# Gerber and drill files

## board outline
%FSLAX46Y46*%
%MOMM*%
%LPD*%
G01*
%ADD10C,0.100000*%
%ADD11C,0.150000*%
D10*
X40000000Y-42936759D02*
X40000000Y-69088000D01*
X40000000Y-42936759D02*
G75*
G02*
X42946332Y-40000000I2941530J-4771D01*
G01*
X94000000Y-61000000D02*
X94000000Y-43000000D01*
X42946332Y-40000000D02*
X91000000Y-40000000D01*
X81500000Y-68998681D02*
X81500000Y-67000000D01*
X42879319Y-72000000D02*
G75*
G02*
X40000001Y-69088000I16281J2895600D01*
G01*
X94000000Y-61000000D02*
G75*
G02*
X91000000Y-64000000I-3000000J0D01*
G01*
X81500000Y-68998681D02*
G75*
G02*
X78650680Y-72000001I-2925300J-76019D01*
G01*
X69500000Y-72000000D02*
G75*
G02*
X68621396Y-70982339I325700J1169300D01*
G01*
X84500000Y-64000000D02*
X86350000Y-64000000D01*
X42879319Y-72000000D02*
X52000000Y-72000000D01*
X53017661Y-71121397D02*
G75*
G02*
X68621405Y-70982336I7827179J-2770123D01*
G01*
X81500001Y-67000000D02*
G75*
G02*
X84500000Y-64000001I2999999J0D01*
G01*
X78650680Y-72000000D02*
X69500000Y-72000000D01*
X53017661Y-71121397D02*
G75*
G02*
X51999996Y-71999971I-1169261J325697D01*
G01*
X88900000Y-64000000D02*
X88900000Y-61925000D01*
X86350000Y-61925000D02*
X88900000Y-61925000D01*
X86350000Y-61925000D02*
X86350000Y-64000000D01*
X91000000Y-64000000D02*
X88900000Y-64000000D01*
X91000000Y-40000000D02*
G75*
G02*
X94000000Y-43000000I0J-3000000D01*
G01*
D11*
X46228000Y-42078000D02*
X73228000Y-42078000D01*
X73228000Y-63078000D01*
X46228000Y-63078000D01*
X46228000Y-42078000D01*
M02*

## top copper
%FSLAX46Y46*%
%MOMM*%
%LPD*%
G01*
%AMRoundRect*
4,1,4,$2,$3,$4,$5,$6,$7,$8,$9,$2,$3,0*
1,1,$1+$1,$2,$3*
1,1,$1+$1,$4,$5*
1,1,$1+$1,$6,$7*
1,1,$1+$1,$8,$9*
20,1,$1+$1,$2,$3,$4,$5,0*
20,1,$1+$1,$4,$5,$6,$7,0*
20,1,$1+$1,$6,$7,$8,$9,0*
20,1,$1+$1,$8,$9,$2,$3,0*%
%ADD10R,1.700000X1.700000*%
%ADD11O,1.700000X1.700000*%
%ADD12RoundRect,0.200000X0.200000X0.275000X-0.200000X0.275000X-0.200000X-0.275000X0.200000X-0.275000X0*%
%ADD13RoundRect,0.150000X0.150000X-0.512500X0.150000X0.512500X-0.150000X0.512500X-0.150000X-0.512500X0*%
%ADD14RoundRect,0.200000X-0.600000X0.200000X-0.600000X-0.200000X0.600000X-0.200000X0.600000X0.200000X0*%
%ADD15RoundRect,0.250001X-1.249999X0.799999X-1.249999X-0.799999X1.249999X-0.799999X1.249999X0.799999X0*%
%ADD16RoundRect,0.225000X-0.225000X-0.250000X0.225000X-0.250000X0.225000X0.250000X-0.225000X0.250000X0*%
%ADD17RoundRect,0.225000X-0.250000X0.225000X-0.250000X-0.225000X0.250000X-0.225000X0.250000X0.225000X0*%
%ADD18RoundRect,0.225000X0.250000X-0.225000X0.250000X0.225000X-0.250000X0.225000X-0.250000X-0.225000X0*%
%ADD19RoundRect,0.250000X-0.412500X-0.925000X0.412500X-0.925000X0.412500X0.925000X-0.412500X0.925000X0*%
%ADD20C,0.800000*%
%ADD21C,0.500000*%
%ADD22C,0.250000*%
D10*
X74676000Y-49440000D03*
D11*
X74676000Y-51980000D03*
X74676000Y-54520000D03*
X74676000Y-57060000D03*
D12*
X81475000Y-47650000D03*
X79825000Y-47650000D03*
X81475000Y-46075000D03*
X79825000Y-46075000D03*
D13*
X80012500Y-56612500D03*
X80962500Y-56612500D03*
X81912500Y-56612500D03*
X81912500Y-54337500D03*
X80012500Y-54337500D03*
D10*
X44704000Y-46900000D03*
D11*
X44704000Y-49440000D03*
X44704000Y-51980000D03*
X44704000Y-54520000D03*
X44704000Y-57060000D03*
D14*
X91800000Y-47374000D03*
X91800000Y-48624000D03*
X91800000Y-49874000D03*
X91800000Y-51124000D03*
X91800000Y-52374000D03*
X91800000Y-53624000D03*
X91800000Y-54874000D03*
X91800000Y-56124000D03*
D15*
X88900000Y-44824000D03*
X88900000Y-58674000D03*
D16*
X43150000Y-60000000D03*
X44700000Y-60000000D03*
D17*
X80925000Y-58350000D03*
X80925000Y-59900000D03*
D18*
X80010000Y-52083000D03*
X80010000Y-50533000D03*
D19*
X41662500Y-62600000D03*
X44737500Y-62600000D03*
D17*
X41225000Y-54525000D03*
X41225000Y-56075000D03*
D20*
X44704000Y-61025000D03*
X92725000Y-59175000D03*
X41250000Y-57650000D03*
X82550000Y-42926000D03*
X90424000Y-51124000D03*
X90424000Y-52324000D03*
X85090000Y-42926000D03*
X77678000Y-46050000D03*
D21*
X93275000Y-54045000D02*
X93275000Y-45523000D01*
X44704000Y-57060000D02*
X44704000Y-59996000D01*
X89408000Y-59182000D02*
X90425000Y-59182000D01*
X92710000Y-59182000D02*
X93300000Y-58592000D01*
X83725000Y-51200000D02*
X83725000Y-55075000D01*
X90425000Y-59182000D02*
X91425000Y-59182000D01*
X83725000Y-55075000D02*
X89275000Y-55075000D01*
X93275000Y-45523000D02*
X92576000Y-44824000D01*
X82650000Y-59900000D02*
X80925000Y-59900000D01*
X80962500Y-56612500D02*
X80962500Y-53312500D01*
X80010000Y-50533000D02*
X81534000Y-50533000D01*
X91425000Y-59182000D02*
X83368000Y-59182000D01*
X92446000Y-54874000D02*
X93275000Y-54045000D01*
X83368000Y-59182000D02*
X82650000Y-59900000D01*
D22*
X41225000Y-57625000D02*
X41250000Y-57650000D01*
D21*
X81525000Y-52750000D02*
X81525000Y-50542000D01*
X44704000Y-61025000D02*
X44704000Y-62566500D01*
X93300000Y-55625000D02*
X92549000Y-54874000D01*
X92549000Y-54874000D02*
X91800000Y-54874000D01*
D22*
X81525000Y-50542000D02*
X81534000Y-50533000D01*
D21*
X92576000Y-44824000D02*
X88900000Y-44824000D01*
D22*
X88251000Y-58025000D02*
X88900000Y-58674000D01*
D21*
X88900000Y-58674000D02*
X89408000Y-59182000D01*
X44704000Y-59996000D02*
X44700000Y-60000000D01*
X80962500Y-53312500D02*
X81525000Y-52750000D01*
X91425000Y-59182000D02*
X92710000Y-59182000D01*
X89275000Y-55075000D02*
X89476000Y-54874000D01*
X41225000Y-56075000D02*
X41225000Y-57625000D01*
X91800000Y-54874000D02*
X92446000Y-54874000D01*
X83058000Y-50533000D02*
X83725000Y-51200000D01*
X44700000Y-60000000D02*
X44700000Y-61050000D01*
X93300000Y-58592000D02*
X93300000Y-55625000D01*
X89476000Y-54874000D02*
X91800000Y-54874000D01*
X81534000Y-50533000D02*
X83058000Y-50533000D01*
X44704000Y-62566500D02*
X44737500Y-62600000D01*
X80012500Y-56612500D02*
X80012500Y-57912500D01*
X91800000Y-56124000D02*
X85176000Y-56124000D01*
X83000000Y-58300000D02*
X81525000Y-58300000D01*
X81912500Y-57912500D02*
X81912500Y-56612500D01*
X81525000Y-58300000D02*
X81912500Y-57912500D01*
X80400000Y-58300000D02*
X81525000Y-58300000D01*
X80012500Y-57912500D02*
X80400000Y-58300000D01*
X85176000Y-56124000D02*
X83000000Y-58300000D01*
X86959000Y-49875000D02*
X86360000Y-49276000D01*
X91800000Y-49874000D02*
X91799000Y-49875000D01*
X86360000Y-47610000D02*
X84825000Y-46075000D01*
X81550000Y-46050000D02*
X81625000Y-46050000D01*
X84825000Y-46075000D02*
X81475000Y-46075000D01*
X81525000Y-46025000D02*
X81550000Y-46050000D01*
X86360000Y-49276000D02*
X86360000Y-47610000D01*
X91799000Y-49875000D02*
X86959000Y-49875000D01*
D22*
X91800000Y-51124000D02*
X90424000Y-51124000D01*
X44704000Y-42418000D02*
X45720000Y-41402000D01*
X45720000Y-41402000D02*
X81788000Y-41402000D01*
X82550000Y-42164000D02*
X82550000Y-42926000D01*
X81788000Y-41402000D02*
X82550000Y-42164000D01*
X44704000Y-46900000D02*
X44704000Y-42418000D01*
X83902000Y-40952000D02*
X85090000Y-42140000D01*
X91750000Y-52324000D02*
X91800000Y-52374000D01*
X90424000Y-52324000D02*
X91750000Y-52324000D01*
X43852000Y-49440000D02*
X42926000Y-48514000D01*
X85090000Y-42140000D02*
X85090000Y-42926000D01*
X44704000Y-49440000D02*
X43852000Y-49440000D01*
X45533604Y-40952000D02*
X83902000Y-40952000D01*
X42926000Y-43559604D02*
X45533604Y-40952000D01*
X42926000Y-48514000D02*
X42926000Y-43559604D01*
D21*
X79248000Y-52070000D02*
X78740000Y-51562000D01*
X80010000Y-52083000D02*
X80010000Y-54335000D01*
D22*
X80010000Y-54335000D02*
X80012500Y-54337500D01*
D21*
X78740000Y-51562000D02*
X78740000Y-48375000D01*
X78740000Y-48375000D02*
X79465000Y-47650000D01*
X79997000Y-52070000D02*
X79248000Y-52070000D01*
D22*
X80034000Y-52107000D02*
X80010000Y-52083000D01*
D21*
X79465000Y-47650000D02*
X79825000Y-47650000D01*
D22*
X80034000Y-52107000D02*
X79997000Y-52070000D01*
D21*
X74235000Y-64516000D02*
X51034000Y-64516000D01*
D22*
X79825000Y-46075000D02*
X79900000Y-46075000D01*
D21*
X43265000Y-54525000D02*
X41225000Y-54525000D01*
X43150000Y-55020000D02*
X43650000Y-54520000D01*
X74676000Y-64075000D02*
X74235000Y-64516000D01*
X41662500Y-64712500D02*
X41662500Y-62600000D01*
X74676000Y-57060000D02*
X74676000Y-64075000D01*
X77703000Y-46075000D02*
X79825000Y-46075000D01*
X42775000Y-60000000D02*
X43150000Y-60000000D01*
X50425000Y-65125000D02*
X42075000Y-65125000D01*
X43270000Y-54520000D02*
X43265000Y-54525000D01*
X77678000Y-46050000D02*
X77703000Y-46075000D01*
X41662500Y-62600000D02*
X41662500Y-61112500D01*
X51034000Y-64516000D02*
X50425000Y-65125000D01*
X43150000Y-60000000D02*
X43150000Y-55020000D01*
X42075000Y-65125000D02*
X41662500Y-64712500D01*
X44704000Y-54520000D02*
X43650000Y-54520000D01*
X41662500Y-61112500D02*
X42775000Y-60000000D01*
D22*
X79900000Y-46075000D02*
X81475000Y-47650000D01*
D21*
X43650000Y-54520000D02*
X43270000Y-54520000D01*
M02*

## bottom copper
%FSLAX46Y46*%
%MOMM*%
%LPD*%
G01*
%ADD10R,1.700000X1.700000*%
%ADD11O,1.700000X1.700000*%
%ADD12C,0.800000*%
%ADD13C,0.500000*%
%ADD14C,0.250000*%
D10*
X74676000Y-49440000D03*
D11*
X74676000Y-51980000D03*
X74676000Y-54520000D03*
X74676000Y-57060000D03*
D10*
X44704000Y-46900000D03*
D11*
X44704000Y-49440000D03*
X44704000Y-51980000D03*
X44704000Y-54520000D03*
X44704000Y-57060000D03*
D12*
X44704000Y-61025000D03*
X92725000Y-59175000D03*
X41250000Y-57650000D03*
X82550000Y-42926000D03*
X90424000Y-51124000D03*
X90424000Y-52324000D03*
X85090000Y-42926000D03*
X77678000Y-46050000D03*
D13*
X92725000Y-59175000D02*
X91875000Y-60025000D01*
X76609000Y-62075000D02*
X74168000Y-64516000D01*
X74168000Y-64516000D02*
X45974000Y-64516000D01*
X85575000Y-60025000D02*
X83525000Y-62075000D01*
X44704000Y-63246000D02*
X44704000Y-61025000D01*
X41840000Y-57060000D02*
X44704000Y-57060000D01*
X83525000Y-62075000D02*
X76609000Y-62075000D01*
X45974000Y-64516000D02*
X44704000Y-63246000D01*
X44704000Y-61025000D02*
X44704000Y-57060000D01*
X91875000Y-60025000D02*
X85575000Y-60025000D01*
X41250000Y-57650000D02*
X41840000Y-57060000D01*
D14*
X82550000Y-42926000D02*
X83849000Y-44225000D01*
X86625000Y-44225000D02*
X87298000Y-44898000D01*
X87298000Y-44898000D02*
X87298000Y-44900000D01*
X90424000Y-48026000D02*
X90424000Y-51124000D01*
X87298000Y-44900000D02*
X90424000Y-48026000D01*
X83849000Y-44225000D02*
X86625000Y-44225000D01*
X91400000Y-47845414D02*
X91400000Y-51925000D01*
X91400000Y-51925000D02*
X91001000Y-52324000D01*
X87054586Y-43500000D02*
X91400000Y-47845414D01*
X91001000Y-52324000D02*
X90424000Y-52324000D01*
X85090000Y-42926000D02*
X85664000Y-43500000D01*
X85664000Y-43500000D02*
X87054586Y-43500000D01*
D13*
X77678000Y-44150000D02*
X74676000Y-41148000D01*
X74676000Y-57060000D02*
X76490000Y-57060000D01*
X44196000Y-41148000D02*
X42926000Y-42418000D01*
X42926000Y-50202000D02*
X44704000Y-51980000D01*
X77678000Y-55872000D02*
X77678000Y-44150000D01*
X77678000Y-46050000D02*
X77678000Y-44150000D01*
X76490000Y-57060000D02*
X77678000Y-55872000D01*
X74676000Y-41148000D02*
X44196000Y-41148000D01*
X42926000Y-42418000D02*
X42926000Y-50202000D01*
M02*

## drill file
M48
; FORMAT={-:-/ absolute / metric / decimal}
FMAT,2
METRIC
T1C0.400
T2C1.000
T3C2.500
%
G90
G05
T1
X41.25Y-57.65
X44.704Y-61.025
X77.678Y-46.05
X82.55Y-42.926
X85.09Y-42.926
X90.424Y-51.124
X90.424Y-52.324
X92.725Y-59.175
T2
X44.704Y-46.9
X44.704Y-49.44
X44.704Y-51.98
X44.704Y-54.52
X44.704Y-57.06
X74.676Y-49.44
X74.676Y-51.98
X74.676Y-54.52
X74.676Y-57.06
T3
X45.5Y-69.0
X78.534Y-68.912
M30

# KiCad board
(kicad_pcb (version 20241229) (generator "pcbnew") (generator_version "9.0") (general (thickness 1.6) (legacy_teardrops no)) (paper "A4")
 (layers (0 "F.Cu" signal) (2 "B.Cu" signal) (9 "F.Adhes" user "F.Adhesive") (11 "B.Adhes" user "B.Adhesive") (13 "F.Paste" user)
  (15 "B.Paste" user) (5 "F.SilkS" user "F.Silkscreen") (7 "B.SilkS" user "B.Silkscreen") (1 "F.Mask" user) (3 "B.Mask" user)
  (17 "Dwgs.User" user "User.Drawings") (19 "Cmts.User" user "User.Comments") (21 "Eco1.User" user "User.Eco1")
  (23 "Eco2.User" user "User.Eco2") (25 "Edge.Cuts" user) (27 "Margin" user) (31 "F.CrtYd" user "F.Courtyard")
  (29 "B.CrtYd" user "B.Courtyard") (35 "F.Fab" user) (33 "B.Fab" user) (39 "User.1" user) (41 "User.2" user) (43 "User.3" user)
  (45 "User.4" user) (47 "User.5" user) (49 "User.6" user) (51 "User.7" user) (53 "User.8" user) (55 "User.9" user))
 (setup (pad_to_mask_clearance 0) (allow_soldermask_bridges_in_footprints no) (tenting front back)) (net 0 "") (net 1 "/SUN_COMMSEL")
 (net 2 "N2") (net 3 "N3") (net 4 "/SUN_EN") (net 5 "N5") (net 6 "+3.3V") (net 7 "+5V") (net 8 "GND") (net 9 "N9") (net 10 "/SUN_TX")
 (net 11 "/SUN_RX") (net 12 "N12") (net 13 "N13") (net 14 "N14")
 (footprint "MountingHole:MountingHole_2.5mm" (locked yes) (layer "F.Cu") (at 45.466 69.088)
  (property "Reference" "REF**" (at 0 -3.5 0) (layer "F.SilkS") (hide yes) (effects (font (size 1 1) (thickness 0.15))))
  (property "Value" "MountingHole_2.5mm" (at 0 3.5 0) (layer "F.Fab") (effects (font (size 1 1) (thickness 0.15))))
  (pad "" np_thru_hole circle (at 0.034 -0.088) (size 2.5 2.5) (drill 2.5) (layers "*.Cu" "*.Mask")))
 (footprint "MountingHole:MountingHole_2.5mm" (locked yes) (layer "F.Cu") (at 78.5 69)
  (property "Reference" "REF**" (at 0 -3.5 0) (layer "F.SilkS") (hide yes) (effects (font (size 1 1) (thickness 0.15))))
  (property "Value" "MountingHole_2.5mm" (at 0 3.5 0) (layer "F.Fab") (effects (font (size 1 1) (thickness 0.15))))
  (pad "" np_thru_hole circle (at 0.034 -0.088) (size 2.5 2.5) (drill 2.5) (layers "*.Cu" "*.Mask")))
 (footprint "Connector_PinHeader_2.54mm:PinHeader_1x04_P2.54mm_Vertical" (layer "F.Cu") (at 74.676 49.44)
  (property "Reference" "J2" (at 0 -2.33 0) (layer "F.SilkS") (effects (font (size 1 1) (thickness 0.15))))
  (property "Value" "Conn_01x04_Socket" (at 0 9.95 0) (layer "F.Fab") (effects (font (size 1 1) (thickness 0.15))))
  (pad "1" thru_hole rect (at 0 0) (size 1.7 1.7) (drill 1) (layers "*.Cu" "*.Mask") (remove_unused_layers no) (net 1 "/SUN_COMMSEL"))
  (pad "2" thru_hole oval (at 0 2.54) (size 1.7 1.7) (drill 1) (layers "*.Cu" "*.Mask") (remove_unused_layers no) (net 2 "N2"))
  (pad "3" thru_hole oval (at 0 5.08) (size 1.7 1.7) (drill 1) (layers "*.Cu" "*.Mask") (remove_unused_layers no) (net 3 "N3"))
  (pad "4" thru_hole oval (at 0 7.62) (size 1.7 1.7) (drill 1) (layers "*.Cu" "*.Mask") (remove_unused_layers no) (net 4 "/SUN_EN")))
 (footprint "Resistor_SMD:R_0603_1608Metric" (layer "F.Cu") (at 80.65 47.65 180)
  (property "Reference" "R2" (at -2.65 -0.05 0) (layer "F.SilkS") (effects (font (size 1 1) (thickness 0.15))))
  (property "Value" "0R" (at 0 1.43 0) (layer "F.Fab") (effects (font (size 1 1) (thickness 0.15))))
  (pad "1" smd roundrect (at -0.825 0 180) (size 0.8 0.95) (layers "F.Cu" "F.Mask" "F.Paste") (roundrect_rratio 0.25) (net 4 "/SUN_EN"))
  (pad "2" smd roundrect (at 0.825 0 180) (size 0.8 0.95) (layers "F.Cu" "F.Mask" "F.Paste") (roundrect_rratio 0.25) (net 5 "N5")))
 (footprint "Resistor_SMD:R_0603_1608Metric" (layer "F.Cu") (at 80.65 46.075 180)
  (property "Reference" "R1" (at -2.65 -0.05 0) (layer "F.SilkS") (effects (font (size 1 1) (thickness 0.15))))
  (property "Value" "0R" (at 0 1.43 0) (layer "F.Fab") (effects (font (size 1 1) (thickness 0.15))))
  (pad "1" smd roundrect (at -0.825 0 180) (size 0.8 0.95) (layers "F.Cu" "F.Mask" "F.Paste") (roundrect_rratio 0.25) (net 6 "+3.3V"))
  (pad "2" smd roundrect (at 0.825 0 180) (size 0.8 0.95) (layers "F.Cu" "F.Mask" "F.Paste") (roundrect_rratio 0.25) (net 4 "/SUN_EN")))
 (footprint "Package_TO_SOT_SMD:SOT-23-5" (layer "F.Cu") (at 80.9625 55.475 90)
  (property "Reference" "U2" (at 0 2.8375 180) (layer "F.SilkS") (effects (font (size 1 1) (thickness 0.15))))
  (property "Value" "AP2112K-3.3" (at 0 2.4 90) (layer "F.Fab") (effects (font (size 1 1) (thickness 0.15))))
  (pad "1" smd roundrect (at -1.1375 -0.95 90) (size 1.325 0.6) (layers "F.Cu" "F.Mask" "F.Paste") (roundrect_rratio 0.25) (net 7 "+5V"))
  (pad "2" smd roundrect (at -1.1375 0 90) (size 1.325 0.6) (layers "F.Cu" "F.Mask" "F.Paste") (roundrect_rratio 0.25) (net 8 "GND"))
  (pad "3" smd roundrect (at -1.1375 0.95 90) (size 1.325 0.6) (layers "F.Cu" "F.Mask" "F.Paste") (roundrect_rratio 0.25) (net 7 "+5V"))
  (pad "4" smd roundrect (at 1.1375 0.95 90) (size 1.325 0.6) (layers "F.Cu" "F.Mask" "F.Paste") (roundrect_rratio 0.25) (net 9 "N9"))
  (pad "5" smd roundrect (at 1.1375 -0.95 90) (size 1.325 0.6) (layers "F.Cu" "F.Mask" "F.Paste") (roundrect_rratio 0.25) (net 5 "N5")))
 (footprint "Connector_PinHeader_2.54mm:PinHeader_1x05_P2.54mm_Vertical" (layer "F.Cu") (at 44.704 46.9)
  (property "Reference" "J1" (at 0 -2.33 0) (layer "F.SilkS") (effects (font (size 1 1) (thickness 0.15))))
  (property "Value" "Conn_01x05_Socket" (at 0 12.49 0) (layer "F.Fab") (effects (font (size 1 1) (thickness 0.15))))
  (pad "1" thru_hole rect (at 0 0) (size 1.7 1.7) (drill 1) (layers "*.Cu" "*.Mask") (remove_unused_layers no) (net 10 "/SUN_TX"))
  (pad "2" thru_hole oval (at 0 2.54) (size 1.7 1.7) (drill 1) (layers "*.Cu" "*.Mask") (remove_unused_layers no) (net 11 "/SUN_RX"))
  (pad "3" thru_hole oval (at 0 5.08) (size 1.7 1.7) (drill 1) (layers "*.Cu" "*.Mask") (remove_unused_layers no) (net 4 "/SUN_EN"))
  (pad "4" thru_hole oval (at 0 7.62) (size 1.7 1.7) (drill 1) (layers "*.Cu" "*.Mask") (remove_unused_layers no) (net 4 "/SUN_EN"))
  (pad "5" thru_hole oval (at 0 10.16) (size 1.7 1.7) (drill 1) (layers "*.Cu" "*.Mask") (remove_unused_layers no) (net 8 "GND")))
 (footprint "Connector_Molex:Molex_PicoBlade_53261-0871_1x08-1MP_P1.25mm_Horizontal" (layer "F.Cu") (at 89.4 51.749 -90)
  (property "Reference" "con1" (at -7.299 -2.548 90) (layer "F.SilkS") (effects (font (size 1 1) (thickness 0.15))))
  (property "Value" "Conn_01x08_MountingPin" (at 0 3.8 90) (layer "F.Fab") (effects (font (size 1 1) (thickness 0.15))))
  (pad "1" smd roundrect (at -4.375 -2.4 270) (size 0.8 1.6) (layers "F.Cu" "F.Mask" "F.Paste") (roundrect_rratio 0.25) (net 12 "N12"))
  (pad "2" smd roundrect (at -3.125 -2.4 270) (size 0.8 1.6) (layers "F.Cu" "F.Mask" "F.Paste") (roundrect_rratio 0.25) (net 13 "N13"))
  (pad "3" smd roundrect (at -1.875 -2.4 270) (size 0.8 1.6) (layers "F.Cu" "F.Mask" "F.Paste") (roundrect_rratio 0.25) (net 6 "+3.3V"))
  (pad "4" smd roundrect (at -0.625 -2.4 270) (size 0.8 1.6) (layers "F.Cu" "F.Mask" "F.Paste") (roundrect_rratio 0.25) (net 10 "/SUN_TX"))
  (pad "5" smd roundrect (at 0.625 -2.4 270) (size 0.8 1.6) (layers "F.Cu" "F.Mask" "F.Paste") (roundrect_rratio 0.25) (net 11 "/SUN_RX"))
  (pad "6" smd roundrect (at 1.875 -2.4 270) (size 0.8 1.6) (layers "F.Cu" "F.Mask" "F.Paste") (roundrect_rratio 0.25) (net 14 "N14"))
  (pad "7" smd roundrect (at 3.125 -2.4 270) (size 0.8 1.6) (layers "F.Cu" "F.Mask" "F.Paste") (roundrect_rratio 0.25) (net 8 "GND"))
  (pad "8" smd roundrect (at 4.375 -2.4 270) (size 0.8 1.6) (layers "F.Cu" "F.Mask" "F.Paste") (roundrect_rratio 0.25) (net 7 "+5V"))
  (pad "MP" smd roundrect (at -6.925 0.5 270) (size 2.1 3) (layers "F.Cu" "F.Mask" "F.Paste") (roundrect_rratio 0.1190480952) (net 8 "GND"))
  (pad "MP" smd roundrect (at 6.925 0.5 270) (size 2.1 3) (layers "F.Cu" "F.Mask" "F.Paste") (roundrect_rratio 0.1190480952) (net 8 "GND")))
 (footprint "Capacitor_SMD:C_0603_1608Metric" (layer "F.Cu") (at 43.925 60)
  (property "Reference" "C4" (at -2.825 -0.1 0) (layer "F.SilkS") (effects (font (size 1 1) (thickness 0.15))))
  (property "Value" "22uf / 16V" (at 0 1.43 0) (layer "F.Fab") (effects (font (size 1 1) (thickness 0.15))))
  (pad "1" smd roundrect (at -0.775 0) (size 0.9 0.95) (layers "F.Cu" "F.Mask" "F.Paste") (roundrect_rratio 0.25) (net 4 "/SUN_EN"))
  (pad "2" smd roundrect (at 0.775 0) (size 0.9 0.95) (layers "F.Cu" "F.Mask" "F.Paste") (roundrect_rratio 0.25) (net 8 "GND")))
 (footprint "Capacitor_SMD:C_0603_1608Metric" (layer "F.Cu") (at 80.925 59.125 -90)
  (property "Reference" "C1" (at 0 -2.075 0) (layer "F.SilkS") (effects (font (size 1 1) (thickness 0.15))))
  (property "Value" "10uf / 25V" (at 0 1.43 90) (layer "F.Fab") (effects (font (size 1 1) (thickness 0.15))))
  (pad "1" smd roundrect (at -0.775 0 270) (size 0.9 0.95) (layers "F.Cu" "F.Mask" "F.Paste") (roundrect_rratio 0.25) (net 7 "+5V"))
  (pad "2" smd roundrect (at 0.775 0 270) (size 0.9 0.95) (layers "F.Cu" "F.Mask" "F.Paste") (roundrect_rratio 0.25) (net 8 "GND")))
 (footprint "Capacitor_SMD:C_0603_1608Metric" (layer "F.Cu") (at 80.01 51.308 90)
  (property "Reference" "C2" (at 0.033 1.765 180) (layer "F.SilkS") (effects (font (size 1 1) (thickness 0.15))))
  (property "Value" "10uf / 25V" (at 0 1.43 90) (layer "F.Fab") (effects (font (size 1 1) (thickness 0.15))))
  (pad "1" smd roundrect (at -0.775 0 90) (size 0.9 0.95) (layers "F.Cu" "F.Mask" "F.Paste") (roundrect_rratio 0.25) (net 5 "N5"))
  (pad "2" smd roundrect (at 0.775 0 90) (size 0.9 0.95) (layers "F.Cu" "F.Mask" "F.Paste") (roundrect_rratio 0.25) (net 8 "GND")))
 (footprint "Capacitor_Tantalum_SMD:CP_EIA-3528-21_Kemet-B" (layer "F.Cu") (at 43.2 62.6)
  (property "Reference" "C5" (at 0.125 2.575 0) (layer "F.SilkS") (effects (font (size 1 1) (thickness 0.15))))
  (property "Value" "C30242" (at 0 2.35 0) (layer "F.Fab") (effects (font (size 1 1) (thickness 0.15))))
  (pad "1" smd roundrect (at -1.5375 0) (size 1.325 2.35) (layers "F.Cu" "F.Mask" "F.Paste") (roundrect_rratio 0.188679) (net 4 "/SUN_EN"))
  (pad "2" smd roundrect (at 1.5375 0) (size 1.325 2.35) (layers "F.Cu" "F.Mask" "F.Paste") (roundrect_rratio 0.188679) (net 8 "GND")))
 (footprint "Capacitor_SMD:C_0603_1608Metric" (layer "F.Cu") (at 41.225 55.3 -90)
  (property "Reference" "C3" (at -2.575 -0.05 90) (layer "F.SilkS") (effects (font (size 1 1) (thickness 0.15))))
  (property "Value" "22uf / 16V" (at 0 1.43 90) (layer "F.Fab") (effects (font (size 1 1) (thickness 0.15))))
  (pad "1" smd roundrect (at -0.775 0 270) (size 0.9 0.95) (layers "F.Cu" "F.Mask" "F.Paste") (roundrect_rratio 0.25) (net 4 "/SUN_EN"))
  (pad "2" smd roundrect (at 0.775 0 270) (size 0.9 0.95) (layers "F.Cu" "F.Mask" "F.Paste") (roundrect_rratio 0.25) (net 8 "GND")))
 (gr_line (start 40 42.936759) (end 40 69.088) (stroke (width 0.1) (type default)) (locked yes) (layer "Edge.Cuts"))
 (gr_arc (start 40 42.936759) (mid 40.864938 40.858169) (end 42.946332 40) (stroke (width 0.1) (type default)) (locked yes)
  (layer "Edge.Cuts"))
 (gr_line (start 94 61) (end 94 43) (stroke (width 0.1) (type default)) (locked yes) (layer "Edge.Cuts"))
 (gr_line (start 42.946332 40) (end 91 40) (stroke (width 0.1) (type default)) (locked yes) (layer "Edge.Cuts"))
 (gr_line (start 81.5 68.998681) (end 81.5 67) (stroke (width 0.1) (type default)) (locked yes) (layer "Edge.Cuts"))
 (gr_arc (start 42.879319 72) (mid 40.83656 71.140332) (end 40 69.088) (stroke (width 0.1) (type default)) (locked yes) (layer "Edge.Cuts"))
 (gr_arc (start 94 61) (mid 93.121321 63.121321) (end 91 64) (stroke (width 0.1) (type default)) (locked yes) (layer "Edge.Cuts"))
 (gr_arc (start 81.5 68.998681) (mid 80.696939 71.089459) (end 78.65068 72) (stroke (width 0.1) (type default)) (locked yes)
  (layer "Edge.Cuts"))
 (gr_arc (start 69.5 72) (mid 68.906927 71.623929) (end 68.621397 70.982339) (stroke (width 0.1) (type default)) (locked yes)
  (layer "Edge.Cuts"))
 (gr_line (start 84.5 64) (end 86.35 64) (stroke (width 0.1) (type default)) (locked yes) (layer "Edge.Cuts"))
 (gr_line (start 42.879319 72) (end 52 72) (stroke (width 0.1) (type default)) (locked yes) (layer "Edge.Cuts"))
 (gr_arc (start 53.017661 71.121397) (mid 60.770843 65.588942) (end 68.621397 70.982339) (stroke (width 0.1) (type default)) (locked yes)
  (layer "Edge.Cuts"))
 (gr_arc (start 81.500001 67) (mid 82.37868 64.878681) (end 84.5 64) (stroke (width 0.1) (type default)) (locked yes) (layer "Edge.Cuts"))
 (gr_line (start 78.65068 72) (end 69.5 72) (stroke (width 0.1) (type default)) (locked yes) (layer "Edge.Cuts"))
 (gr_arc (start 53.017661 71.121397) (mid 52.64159 71.71447) (end 52 72) (stroke (width 0.1) (type default)) (locked yes)
  (layer "Edge.Cuts"))
 (gr_line (start 88.9 64) (end 88.9 61.925) (stroke (width 0.1) (type default)) (locked yes) (layer "Edge.Cuts"))
 (gr_line (start 86.35 61.925) (end 88.9 61.925) (stroke (width 0.1) (type default)) (locked yes) (layer "Edge.Cuts"))
 (gr_line (start 86.35 61.925) (end 86.35 64) (stroke (width 0.1) (type default)) (locked yes) (layer "Edge.Cuts"))
 (gr_line (start 91 64) (end 88.9 64) (stroke (width 0.1) (type default)) (locked yes) (layer "Edge.Cuts"))
 (gr_arc (start 91 40) (mid 93.121321 40.878679) (end 94 43) (stroke (width 0.1) (type default)) (locked yes) (layer "Edge.Cuts"))
 (gr_rect (start 46.228 42.078) (end 73.228 63.078) (stroke (width 0.15) (type default)) (fill no) (locked yes) (layer "Edge.Cuts"))
 (segment (start 93.275 54.045) (end 93.275 45.523) (width 0.5) (layer "F.Cu") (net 8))
 (segment (start 44.704 57.06) (end 44.704 59.996) (width 0.5) (layer "F.Cu") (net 8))
 (segment (start 89.408 59.182) (end 90.425 59.182) (width 0.5) (layer "F.Cu") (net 8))
 (segment (start 92.71 59.182) (end 93.3 58.592) (width 0.5) (layer "F.Cu") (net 8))
 (segment (start 83.725 51.2) (end 83.725 55.075) (width 0.5) (layer "F.Cu") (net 8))
 (segment (start 90.425 59.182) (end 91.425 59.182) (width 0.5) (layer "F.Cu") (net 8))
 (segment (start 83.725 55.075) (end 89.275 55.075) (width 0.5) (layer "F.Cu") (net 8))
 (segment (start 93.275 45.523) (end 92.576 44.824) (width 0.5) (layer "F.Cu") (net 8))
 (segment (start 82.65 59.9) (end 80.925 59.9) (width 0.5) (layer "F.Cu") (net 8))
 (segment (start 80.9625 56.6125) (end 80.9625 53.3125) (width 0.5) (layer "F.Cu") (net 8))
 (segment (start 80.01 50.533) (end 81.534 50.533) (width 0.5) (layer "F.Cu") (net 8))
 (segment (start 91.425 59.182) (end 83.368 59.182) (width 0.5) (layer "F.Cu") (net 8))
 (segment (start 92.446 54.874) (end 93.275 54.045) (width 0.5) (layer "F.Cu") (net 8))
 (segment (start 83.368 59.182) (end 82.65 59.9) (width 0.5) (layer "F.Cu") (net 8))
 (segment (start 41.225 57.625) (end 41.25 57.65) (width 0.25) (layer "F.Cu") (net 8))
 (segment (start 81.525 52.75) (end 81.525 50.542) (width 0.5) (layer "F.Cu") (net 8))
 (segment (start 44.704 61.025) (end 44.704 62.5665) (width 0.5) (layer "F.Cu") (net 8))
 (segment (start 93.3 55.625) (end 92.549 54.874) (width 0.5) (layer "F.Cu") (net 8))
 (segment (start 92.549 54.874) (end 91.8 54.874) (width 0.5) (layer "F.Cu") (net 8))
 (segment (start 81.525 50.542) (end 81.534 50.533) (width 0.25) (layer "F.Cu") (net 8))
 (segment (start 92.576 44.824) (end 88.9 44.824) (width 0.5) (layer "F.Cu") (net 8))
 (segment (start 88.251 58.025) (end 88.9 58.674) (width 0.25) (layer "F.Cu") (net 8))
 (segment (start 88.9 58.674) (end 89.408 59.182) (width 0.5) (layer "F.Cu") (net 8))
 (segment (start 44.704 59.996) (end 44.7 60) (width 0.5) (layer "F.Cu") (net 8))
 (segment (start 80.9625 53.3125) (end 81.525 52.75) (width 0.5) (layer "F.Cu") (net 8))
 (segment (start 91.425 59.182) (end 92.71 59.182) (width 0.5) (layer "F.Cu") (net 8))
 (segment (start 89.275 55.075) (end 89.476 54.874) (width 0.5) (layer "F.Cu") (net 8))
 (segment (start 41.225 56.075) (end 41.225 57.625) (width 0.5) (layer "F.Cu") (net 8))
 (segment (start 91.8 54.874) (end 92.446 54.874) (width 0.5) (layer "F.Cu") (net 8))
 (segment (start 83.058 50.533) (end 83.725 51.2) (width 0.5) (layer "F.Cu") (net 8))
 (segment (start 44.7 60) (end 44.7 61.05) (width 0.5) (layer "F.Cu") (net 8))
 (segment (start 93.3 58.592) (end 93.3 55.625) (width 0.5) (layer "F.Cu") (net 8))
 (segment (start 89.476 54.874) (end 91.8 54.874) (width 0.5) (layer "F.Cu") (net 8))
 (segment (start 81.534 50.533) (end 83.058 50.533) (width 0.5) (layer "F.Cu") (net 8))
 (segment (start 44.704 62.5665) (end 44.7375 62.6) (width 0.5) (layer "F.Cu") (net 8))
 (via (at 44.704 61.025) (size 0.8) (drill 0.4) (layers "F.Cu" "B.Cu") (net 8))
 (via (at 92.725 59.175) (size 0.8) (drill 0.4) (layers "F.Cu" "B.Cu") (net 8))
 (via (at 41.25 57.65) (size 0.8) (drill 0.4) (layers "F.Cu" "B.Cu") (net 8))
 (segment (start 92.725 59.175) (end 91.875 60.025) (width 0.5) (layer "B.Cu") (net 8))
 (segment (start 76.609 62.075) (end 74.168 64.516) (width 0.5) (layer "B.Cu") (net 8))
 (segment (start 74.168 64.516) (end 45.974 64.516) (width 0.5) (layer "B.Cu") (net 8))
 (segment (start 85.575 60.025) (end 83.525 62.075) (width 0.5) (layer "B.Cu") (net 8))
 (segment (start 44.704 63.246) (end 44.704 61.025) (width 0.5) (layer "B.Cu") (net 8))
 (segment (start 41.84 57.06) (end 44.704 57.06) (width 0.5) (layer "B.Cu") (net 8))
 (segment (start 83.525 62.075) (end 76.609 62.075) (width 0.5) (layer "B.Cu") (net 8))
 (segment (start 45.974 64.516) (end 44.704 63.246) (width 0.5) (layer "B.Cu") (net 8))
 (segment (start 44.704 61.025) (end 44.704 57.06) (width 0.5) (layer "B.Cu") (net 8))
 (segment (start 91.875 60.025) (end 85.575 60.025) (width 0.5) (layer "B.Cu") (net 8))
 (segment (start 41.25 57.65) (end 41.84 57.06) (width 0.5) (layer "B.Cu") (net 8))
 (segment (start 80.0125 56.6125) (end 80.0125 57.9125) (width 0.5) (layer "F.Cu") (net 7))
 (segment (start 91.8 56.124) (end 85.176 56.124) (width 0.5) (layer "F.Cu") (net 7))
 (segment (start 83 58.3) (end 81.525 58.3) (width 0.5) (layer "F.Cu") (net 7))
 (segment (start 81.9125 57.9125) (end 81.9125 56.6125) (width 0.5) (layer "F.Cu") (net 7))
 (segment (start 81.525 58.3) (end 81.9125 57.9125) (width 0.5) (layer "F.Cu") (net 7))
 (segment (start 80.4 58.3) (end 81.525 58.3) (width 0.5) (layer "F.Cu") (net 7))
 (segment (start 80.0125 57.9125) (end 80.4 58.3) (width 0.5) (layer "F.Cu") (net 7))
 (segment (start 85.176 56.124) (end 83 58.3) (width 0.5) (layer "F.Cu") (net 7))
 (segment (start 86.959 49.875) (end 86.36 49.276) (width 0.5) (layer "F.Cu") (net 6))
 (segment (start 91.8 49.874) (end 91.799 49.875) (width 0.5) (layer "F.Cu") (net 6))
 (segment (start 86.36 47.61) (end 84.825 46.075) (width 0.5) (layer "F.Cu") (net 6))
 (segment (start 81.55 46.05) (end 81.625 46.05) (width 0.5) (layer "F.Cu") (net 6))
 (segment (start 84.825 46.075) (end 81.475 46.075) (width 0.5) (layer "F.Cu") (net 6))
 (segment (start 81.525 46.025) (end 81.55 46.05) (width 0.5) (layer "F.Cu") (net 6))
 (segment (start 86.36 49.276) (end 86.36 47.61) (width 0.5) (layer "F.Cu") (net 6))
 (segment (start 91.799 49.875) (end 86.959 49.875) (width 0.5) (layer "F.Cu") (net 6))
 (segment (start 91.8 51.124) (end 90.424 51.124) (width 0.25) (layer "F.Cu") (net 10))
 (segment (start 44.704 42.418) (end 45.72 41.402) (width 0.25) (layer "F.Cu") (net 10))
 (segment (start 45.72 41.402) (end 81.788 41.402) (width 0.25) (layer "F.Cu") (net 10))
 (segment (start 82.55 42.164) (end 82.55 42.926) (width 0.25) (layer "F.Cu") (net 10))
 (segment (start 81.788 41.402) (end 82.55 42.164) (width 0.25) (layer "F.Cu") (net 10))
 (segment (start 44.704 46.9) (end 44.704 42.418) (width 0.25) (layer "F.Cu") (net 10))
 (via (at 82.55 42.926) (size 0.8) (drill 0.4) (layers "F.Cu" "B.Cu") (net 10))
 (via (at 90.424 51.124) (size 0.8) (drill 0.4) (layers "F.Cu" "B.Cu") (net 10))
 (segment (start 82.55 42.926) (end 83.849 44.225) (width 0.25) (layer "B.Cu") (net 10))
 (segment (start 86.625 44.225) (end 87.298 44.898) (width 0.25) (layer "B.Cu") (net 10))
 (segment (start 87.298 44.898) (end 87.298 44.9) (width 0.25) (layer "B.Cu") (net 10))
 (segment (start 90.424 48.026) (end 90.424 51.124) (width 0.25) (layer "B.Cu") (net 10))
 (segment (start 87.298 44.9) (end 90.424 48.026) (width 0.25) (layer "B.Cu") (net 10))
 (segment (start 83.849 44.225) (end 86.625 44.225) (width 0.25) (layer "B.Cu") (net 10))
 (segment (start 83.902 40.952) (end 85.09 42.14) (width 0.25) (layer "F.Cu") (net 11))
 (segment (start 91.75 52.324) (end 91.8 52.374) (width 0.25) (layer "F.Cu") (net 11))
 (segment (start 90.424 52.324) (end 91.75 52.324) (width 0.25) (layer "F.Cu") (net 11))
 (segment (start 43.852 49.44) (end 42.926 48.514) (width 0.25) (layer "F.Cu") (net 11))
 (segment (start 85.09 42.14) (end 85.09 42.926) (width 0.25) (layer "F.Cu") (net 11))
 (segment (start 44.704 49.44) (end 43.852 49.44) (width 0.25) (layer "F.Cu") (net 11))
 (segment (start 45.533604 40.952) (end 83.902 40.952) (width 0.25) (layer "F.Cu") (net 11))
 (segment (start 42.926 43.559604) (end 45.533604 40.952) (width 0.25) (layer "F.Cu") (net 11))
 (segment (start 42.926 48.514) (end 42.926 43.559604) (width 0.25) (layer "F.Cu") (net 11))
 (via (at 90.424 52.324) (size 0.8) (drill 0.4) (layers "F.Cu" "B.Cu") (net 11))
 (via (at 85.09 42.926) (size 0.8) (drill 0.4) (layers "F.Cu" "B.Cu") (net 11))
 (segment (start 91.4 47.845414) (end 91.4 51.925) (width 0.25) (layer "B.Cu") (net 11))
 (segment (start 91.4 51.925) (end 91.001 52.324) (width 0.25) (layer "B.Cu") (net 11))
 (segment (start 87.054586 43.5) (end 91.4 47.845414) (width 0.25) (layer "B.Cu") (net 11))
 (segment (start 91.001 52.324) (end 90.424 52.324) (width 0.25) (layer "B.Cu") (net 11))
 (segment (start 85.09 42.926) (end 85.664 43.5) (width 0.25) (layer "B.Cu") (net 11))
 (segment (start 85.664 43.5) (end 87.054586 43.5) (width 0.25) (layer "B.Cu") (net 11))
 (segment (start 79.248 52.07) (end 78.74 51.562) (width 0.5) (layer "F.Cu") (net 5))
 (segment (start 80.01 52.083) (end 80.01 54.335) (width 0.5) (layer "F.Cu") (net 5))
 (segment (start 80.01 54.335) (end 80.0125 54.3375) (width 0.25) (layer "F.Cu") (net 5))
 (segment (start 78.74 51.562) (end 78.74 48.375) (width 0.5) (layer "F.Cu") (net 5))
 (segment (start 78.74 48.375) (end 79.465 47.65) (width 0.5) (layer "F.Cu") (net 5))
 (segment (start 79.997 52.07) (end 79.248 52.07) (width 0.5) (layer "F.Cu") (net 5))
 (segment (start 80.034 52.107) (end 80.01 52.083) (width 0.25) (layer "F.Cu") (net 5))
 (segment (start 79.465 47.65) (end 79.825 47.65) (width 0.5) (layer "F.Cu") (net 5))
 (segment (start 80.034 52.107) (end 79.997 52.07) (width 0.25) (layer "F.Cu") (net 5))
 (segment (start 74.235 64.516) (end 51.034 64.516) (width 0.5) (layer "F.Cu") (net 4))
 (segment (start 79.825 46.075) (end 79.9 46.075) (width 0.25) (layer "F.Cu") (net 4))
 (segment (start 43.265 54.525) (end 41.225 54.525) (width 0.5) (layer "F.Cu") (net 4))
 (segment (start 43.15 55.02) (end 43.65 54.52) (width 0.5) (layer "F.Cu") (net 4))
 (segment (start 74.676 64.075) (end 74.235 64.516) (width 0.5) (layer "F.Cu") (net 4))
 (segment (start 41.6625 64.7125) (end 41.6625 62.6) (width 0.5) (layer "F.Cu") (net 4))
 (segment (start 74.676 57.06) (end 74.676 64.075) (width 0.5) (layer "F.Cu") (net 4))
 (segment (start 77.703 46.075) (end 79.825 46.075) (width 0.5) (layer "F.Cu") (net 4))
 (segment (start 42.775 60) (end 43.15 60) (width 0.5) (layer "F.Cu") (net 4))
 (segment (start 50.425 65.125) (end 42.075 65.125) (width 0.5) (layer "F.Cu") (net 4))
 (segment (start 43.27 54.52) (end 43.265 54.525) (width 0.5) (layer "F.Cu") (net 4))
 (segment (start 77.678 46.05) (end 77.703 46.075) (width 0.5) (layer "F.Cu") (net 4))
 (segment (start 41.6625 62.6) (end 41.6625 61.1125) (width 0.5) (layer "F.Cu") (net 4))
 (segment (start 51.034 64.516) (end 50.425 65.125) (width 0.5) (layer "F.Cu") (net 4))
 (segment (start 43.15 60) (end 43.15 55.02) (width 0.5) (layer "F.Cu") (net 4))
 (segment (start 42.075 65.125) (end 41.6625 64.7125) (width 0.5) (layer "F.Cu") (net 4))
 (segment (start 44.704 54.52) (end 43.65 54.52) (width 0.5) (layer "F.Cu") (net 4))
 (segment (start 41.6625 61.1125) (end 42.775 60) (width 0.5) (layer "F.Cu") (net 4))
 (segment (start 79.9 46.075) (end 81.475 47.65) (width 0.25) (layer "F.Cu") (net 4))
 (segment (start 43.65 54.52) (end 43.27 54.52) (width 0.5) (layer "F.Cu") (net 4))
 (via (at 77.678 46.05) (size 0.8) (drill 0.4) (layers "F.Cu" "B.Cu") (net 4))
 (segment (start 77.678 44.15) (end 74.676 41.148) (width 0.5) (layer "B.Cu") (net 4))
 (segment (start 74.676 57.06) (end 76.49 57.06) (width 0.5) (layer "B.Cu") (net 4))
 (segment (start 44.196 41.148) (end 42.926 42.418) (width 0.5) (layer "B.Cu") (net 4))
 (segment (start 42.926 50.202) (end 44.704 51.98) (width 0.5) (layer "B.Cu") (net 4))
 (segment (start 77.678 55.872) (end 77.678 44.15) (width 0.5) (layer "B.Cu") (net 4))
 (segment (start 77.678 46.05) (end 77.678 44.15) (width 0.5) (layer "B.Cu") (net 4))
 (segment (start 76.49 57.06) (end 77.678 55.872) (width 0.5) (layer "B.Cu") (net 4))
 (segment (start 74.676 41.148) (end 44.196 41.148) (width 0.5) (layer "B.Cu") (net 4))
 (segment (start 42.926 42.418) (end 42.926 50.202) (width 0.5) (layer "B.Cu") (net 4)))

